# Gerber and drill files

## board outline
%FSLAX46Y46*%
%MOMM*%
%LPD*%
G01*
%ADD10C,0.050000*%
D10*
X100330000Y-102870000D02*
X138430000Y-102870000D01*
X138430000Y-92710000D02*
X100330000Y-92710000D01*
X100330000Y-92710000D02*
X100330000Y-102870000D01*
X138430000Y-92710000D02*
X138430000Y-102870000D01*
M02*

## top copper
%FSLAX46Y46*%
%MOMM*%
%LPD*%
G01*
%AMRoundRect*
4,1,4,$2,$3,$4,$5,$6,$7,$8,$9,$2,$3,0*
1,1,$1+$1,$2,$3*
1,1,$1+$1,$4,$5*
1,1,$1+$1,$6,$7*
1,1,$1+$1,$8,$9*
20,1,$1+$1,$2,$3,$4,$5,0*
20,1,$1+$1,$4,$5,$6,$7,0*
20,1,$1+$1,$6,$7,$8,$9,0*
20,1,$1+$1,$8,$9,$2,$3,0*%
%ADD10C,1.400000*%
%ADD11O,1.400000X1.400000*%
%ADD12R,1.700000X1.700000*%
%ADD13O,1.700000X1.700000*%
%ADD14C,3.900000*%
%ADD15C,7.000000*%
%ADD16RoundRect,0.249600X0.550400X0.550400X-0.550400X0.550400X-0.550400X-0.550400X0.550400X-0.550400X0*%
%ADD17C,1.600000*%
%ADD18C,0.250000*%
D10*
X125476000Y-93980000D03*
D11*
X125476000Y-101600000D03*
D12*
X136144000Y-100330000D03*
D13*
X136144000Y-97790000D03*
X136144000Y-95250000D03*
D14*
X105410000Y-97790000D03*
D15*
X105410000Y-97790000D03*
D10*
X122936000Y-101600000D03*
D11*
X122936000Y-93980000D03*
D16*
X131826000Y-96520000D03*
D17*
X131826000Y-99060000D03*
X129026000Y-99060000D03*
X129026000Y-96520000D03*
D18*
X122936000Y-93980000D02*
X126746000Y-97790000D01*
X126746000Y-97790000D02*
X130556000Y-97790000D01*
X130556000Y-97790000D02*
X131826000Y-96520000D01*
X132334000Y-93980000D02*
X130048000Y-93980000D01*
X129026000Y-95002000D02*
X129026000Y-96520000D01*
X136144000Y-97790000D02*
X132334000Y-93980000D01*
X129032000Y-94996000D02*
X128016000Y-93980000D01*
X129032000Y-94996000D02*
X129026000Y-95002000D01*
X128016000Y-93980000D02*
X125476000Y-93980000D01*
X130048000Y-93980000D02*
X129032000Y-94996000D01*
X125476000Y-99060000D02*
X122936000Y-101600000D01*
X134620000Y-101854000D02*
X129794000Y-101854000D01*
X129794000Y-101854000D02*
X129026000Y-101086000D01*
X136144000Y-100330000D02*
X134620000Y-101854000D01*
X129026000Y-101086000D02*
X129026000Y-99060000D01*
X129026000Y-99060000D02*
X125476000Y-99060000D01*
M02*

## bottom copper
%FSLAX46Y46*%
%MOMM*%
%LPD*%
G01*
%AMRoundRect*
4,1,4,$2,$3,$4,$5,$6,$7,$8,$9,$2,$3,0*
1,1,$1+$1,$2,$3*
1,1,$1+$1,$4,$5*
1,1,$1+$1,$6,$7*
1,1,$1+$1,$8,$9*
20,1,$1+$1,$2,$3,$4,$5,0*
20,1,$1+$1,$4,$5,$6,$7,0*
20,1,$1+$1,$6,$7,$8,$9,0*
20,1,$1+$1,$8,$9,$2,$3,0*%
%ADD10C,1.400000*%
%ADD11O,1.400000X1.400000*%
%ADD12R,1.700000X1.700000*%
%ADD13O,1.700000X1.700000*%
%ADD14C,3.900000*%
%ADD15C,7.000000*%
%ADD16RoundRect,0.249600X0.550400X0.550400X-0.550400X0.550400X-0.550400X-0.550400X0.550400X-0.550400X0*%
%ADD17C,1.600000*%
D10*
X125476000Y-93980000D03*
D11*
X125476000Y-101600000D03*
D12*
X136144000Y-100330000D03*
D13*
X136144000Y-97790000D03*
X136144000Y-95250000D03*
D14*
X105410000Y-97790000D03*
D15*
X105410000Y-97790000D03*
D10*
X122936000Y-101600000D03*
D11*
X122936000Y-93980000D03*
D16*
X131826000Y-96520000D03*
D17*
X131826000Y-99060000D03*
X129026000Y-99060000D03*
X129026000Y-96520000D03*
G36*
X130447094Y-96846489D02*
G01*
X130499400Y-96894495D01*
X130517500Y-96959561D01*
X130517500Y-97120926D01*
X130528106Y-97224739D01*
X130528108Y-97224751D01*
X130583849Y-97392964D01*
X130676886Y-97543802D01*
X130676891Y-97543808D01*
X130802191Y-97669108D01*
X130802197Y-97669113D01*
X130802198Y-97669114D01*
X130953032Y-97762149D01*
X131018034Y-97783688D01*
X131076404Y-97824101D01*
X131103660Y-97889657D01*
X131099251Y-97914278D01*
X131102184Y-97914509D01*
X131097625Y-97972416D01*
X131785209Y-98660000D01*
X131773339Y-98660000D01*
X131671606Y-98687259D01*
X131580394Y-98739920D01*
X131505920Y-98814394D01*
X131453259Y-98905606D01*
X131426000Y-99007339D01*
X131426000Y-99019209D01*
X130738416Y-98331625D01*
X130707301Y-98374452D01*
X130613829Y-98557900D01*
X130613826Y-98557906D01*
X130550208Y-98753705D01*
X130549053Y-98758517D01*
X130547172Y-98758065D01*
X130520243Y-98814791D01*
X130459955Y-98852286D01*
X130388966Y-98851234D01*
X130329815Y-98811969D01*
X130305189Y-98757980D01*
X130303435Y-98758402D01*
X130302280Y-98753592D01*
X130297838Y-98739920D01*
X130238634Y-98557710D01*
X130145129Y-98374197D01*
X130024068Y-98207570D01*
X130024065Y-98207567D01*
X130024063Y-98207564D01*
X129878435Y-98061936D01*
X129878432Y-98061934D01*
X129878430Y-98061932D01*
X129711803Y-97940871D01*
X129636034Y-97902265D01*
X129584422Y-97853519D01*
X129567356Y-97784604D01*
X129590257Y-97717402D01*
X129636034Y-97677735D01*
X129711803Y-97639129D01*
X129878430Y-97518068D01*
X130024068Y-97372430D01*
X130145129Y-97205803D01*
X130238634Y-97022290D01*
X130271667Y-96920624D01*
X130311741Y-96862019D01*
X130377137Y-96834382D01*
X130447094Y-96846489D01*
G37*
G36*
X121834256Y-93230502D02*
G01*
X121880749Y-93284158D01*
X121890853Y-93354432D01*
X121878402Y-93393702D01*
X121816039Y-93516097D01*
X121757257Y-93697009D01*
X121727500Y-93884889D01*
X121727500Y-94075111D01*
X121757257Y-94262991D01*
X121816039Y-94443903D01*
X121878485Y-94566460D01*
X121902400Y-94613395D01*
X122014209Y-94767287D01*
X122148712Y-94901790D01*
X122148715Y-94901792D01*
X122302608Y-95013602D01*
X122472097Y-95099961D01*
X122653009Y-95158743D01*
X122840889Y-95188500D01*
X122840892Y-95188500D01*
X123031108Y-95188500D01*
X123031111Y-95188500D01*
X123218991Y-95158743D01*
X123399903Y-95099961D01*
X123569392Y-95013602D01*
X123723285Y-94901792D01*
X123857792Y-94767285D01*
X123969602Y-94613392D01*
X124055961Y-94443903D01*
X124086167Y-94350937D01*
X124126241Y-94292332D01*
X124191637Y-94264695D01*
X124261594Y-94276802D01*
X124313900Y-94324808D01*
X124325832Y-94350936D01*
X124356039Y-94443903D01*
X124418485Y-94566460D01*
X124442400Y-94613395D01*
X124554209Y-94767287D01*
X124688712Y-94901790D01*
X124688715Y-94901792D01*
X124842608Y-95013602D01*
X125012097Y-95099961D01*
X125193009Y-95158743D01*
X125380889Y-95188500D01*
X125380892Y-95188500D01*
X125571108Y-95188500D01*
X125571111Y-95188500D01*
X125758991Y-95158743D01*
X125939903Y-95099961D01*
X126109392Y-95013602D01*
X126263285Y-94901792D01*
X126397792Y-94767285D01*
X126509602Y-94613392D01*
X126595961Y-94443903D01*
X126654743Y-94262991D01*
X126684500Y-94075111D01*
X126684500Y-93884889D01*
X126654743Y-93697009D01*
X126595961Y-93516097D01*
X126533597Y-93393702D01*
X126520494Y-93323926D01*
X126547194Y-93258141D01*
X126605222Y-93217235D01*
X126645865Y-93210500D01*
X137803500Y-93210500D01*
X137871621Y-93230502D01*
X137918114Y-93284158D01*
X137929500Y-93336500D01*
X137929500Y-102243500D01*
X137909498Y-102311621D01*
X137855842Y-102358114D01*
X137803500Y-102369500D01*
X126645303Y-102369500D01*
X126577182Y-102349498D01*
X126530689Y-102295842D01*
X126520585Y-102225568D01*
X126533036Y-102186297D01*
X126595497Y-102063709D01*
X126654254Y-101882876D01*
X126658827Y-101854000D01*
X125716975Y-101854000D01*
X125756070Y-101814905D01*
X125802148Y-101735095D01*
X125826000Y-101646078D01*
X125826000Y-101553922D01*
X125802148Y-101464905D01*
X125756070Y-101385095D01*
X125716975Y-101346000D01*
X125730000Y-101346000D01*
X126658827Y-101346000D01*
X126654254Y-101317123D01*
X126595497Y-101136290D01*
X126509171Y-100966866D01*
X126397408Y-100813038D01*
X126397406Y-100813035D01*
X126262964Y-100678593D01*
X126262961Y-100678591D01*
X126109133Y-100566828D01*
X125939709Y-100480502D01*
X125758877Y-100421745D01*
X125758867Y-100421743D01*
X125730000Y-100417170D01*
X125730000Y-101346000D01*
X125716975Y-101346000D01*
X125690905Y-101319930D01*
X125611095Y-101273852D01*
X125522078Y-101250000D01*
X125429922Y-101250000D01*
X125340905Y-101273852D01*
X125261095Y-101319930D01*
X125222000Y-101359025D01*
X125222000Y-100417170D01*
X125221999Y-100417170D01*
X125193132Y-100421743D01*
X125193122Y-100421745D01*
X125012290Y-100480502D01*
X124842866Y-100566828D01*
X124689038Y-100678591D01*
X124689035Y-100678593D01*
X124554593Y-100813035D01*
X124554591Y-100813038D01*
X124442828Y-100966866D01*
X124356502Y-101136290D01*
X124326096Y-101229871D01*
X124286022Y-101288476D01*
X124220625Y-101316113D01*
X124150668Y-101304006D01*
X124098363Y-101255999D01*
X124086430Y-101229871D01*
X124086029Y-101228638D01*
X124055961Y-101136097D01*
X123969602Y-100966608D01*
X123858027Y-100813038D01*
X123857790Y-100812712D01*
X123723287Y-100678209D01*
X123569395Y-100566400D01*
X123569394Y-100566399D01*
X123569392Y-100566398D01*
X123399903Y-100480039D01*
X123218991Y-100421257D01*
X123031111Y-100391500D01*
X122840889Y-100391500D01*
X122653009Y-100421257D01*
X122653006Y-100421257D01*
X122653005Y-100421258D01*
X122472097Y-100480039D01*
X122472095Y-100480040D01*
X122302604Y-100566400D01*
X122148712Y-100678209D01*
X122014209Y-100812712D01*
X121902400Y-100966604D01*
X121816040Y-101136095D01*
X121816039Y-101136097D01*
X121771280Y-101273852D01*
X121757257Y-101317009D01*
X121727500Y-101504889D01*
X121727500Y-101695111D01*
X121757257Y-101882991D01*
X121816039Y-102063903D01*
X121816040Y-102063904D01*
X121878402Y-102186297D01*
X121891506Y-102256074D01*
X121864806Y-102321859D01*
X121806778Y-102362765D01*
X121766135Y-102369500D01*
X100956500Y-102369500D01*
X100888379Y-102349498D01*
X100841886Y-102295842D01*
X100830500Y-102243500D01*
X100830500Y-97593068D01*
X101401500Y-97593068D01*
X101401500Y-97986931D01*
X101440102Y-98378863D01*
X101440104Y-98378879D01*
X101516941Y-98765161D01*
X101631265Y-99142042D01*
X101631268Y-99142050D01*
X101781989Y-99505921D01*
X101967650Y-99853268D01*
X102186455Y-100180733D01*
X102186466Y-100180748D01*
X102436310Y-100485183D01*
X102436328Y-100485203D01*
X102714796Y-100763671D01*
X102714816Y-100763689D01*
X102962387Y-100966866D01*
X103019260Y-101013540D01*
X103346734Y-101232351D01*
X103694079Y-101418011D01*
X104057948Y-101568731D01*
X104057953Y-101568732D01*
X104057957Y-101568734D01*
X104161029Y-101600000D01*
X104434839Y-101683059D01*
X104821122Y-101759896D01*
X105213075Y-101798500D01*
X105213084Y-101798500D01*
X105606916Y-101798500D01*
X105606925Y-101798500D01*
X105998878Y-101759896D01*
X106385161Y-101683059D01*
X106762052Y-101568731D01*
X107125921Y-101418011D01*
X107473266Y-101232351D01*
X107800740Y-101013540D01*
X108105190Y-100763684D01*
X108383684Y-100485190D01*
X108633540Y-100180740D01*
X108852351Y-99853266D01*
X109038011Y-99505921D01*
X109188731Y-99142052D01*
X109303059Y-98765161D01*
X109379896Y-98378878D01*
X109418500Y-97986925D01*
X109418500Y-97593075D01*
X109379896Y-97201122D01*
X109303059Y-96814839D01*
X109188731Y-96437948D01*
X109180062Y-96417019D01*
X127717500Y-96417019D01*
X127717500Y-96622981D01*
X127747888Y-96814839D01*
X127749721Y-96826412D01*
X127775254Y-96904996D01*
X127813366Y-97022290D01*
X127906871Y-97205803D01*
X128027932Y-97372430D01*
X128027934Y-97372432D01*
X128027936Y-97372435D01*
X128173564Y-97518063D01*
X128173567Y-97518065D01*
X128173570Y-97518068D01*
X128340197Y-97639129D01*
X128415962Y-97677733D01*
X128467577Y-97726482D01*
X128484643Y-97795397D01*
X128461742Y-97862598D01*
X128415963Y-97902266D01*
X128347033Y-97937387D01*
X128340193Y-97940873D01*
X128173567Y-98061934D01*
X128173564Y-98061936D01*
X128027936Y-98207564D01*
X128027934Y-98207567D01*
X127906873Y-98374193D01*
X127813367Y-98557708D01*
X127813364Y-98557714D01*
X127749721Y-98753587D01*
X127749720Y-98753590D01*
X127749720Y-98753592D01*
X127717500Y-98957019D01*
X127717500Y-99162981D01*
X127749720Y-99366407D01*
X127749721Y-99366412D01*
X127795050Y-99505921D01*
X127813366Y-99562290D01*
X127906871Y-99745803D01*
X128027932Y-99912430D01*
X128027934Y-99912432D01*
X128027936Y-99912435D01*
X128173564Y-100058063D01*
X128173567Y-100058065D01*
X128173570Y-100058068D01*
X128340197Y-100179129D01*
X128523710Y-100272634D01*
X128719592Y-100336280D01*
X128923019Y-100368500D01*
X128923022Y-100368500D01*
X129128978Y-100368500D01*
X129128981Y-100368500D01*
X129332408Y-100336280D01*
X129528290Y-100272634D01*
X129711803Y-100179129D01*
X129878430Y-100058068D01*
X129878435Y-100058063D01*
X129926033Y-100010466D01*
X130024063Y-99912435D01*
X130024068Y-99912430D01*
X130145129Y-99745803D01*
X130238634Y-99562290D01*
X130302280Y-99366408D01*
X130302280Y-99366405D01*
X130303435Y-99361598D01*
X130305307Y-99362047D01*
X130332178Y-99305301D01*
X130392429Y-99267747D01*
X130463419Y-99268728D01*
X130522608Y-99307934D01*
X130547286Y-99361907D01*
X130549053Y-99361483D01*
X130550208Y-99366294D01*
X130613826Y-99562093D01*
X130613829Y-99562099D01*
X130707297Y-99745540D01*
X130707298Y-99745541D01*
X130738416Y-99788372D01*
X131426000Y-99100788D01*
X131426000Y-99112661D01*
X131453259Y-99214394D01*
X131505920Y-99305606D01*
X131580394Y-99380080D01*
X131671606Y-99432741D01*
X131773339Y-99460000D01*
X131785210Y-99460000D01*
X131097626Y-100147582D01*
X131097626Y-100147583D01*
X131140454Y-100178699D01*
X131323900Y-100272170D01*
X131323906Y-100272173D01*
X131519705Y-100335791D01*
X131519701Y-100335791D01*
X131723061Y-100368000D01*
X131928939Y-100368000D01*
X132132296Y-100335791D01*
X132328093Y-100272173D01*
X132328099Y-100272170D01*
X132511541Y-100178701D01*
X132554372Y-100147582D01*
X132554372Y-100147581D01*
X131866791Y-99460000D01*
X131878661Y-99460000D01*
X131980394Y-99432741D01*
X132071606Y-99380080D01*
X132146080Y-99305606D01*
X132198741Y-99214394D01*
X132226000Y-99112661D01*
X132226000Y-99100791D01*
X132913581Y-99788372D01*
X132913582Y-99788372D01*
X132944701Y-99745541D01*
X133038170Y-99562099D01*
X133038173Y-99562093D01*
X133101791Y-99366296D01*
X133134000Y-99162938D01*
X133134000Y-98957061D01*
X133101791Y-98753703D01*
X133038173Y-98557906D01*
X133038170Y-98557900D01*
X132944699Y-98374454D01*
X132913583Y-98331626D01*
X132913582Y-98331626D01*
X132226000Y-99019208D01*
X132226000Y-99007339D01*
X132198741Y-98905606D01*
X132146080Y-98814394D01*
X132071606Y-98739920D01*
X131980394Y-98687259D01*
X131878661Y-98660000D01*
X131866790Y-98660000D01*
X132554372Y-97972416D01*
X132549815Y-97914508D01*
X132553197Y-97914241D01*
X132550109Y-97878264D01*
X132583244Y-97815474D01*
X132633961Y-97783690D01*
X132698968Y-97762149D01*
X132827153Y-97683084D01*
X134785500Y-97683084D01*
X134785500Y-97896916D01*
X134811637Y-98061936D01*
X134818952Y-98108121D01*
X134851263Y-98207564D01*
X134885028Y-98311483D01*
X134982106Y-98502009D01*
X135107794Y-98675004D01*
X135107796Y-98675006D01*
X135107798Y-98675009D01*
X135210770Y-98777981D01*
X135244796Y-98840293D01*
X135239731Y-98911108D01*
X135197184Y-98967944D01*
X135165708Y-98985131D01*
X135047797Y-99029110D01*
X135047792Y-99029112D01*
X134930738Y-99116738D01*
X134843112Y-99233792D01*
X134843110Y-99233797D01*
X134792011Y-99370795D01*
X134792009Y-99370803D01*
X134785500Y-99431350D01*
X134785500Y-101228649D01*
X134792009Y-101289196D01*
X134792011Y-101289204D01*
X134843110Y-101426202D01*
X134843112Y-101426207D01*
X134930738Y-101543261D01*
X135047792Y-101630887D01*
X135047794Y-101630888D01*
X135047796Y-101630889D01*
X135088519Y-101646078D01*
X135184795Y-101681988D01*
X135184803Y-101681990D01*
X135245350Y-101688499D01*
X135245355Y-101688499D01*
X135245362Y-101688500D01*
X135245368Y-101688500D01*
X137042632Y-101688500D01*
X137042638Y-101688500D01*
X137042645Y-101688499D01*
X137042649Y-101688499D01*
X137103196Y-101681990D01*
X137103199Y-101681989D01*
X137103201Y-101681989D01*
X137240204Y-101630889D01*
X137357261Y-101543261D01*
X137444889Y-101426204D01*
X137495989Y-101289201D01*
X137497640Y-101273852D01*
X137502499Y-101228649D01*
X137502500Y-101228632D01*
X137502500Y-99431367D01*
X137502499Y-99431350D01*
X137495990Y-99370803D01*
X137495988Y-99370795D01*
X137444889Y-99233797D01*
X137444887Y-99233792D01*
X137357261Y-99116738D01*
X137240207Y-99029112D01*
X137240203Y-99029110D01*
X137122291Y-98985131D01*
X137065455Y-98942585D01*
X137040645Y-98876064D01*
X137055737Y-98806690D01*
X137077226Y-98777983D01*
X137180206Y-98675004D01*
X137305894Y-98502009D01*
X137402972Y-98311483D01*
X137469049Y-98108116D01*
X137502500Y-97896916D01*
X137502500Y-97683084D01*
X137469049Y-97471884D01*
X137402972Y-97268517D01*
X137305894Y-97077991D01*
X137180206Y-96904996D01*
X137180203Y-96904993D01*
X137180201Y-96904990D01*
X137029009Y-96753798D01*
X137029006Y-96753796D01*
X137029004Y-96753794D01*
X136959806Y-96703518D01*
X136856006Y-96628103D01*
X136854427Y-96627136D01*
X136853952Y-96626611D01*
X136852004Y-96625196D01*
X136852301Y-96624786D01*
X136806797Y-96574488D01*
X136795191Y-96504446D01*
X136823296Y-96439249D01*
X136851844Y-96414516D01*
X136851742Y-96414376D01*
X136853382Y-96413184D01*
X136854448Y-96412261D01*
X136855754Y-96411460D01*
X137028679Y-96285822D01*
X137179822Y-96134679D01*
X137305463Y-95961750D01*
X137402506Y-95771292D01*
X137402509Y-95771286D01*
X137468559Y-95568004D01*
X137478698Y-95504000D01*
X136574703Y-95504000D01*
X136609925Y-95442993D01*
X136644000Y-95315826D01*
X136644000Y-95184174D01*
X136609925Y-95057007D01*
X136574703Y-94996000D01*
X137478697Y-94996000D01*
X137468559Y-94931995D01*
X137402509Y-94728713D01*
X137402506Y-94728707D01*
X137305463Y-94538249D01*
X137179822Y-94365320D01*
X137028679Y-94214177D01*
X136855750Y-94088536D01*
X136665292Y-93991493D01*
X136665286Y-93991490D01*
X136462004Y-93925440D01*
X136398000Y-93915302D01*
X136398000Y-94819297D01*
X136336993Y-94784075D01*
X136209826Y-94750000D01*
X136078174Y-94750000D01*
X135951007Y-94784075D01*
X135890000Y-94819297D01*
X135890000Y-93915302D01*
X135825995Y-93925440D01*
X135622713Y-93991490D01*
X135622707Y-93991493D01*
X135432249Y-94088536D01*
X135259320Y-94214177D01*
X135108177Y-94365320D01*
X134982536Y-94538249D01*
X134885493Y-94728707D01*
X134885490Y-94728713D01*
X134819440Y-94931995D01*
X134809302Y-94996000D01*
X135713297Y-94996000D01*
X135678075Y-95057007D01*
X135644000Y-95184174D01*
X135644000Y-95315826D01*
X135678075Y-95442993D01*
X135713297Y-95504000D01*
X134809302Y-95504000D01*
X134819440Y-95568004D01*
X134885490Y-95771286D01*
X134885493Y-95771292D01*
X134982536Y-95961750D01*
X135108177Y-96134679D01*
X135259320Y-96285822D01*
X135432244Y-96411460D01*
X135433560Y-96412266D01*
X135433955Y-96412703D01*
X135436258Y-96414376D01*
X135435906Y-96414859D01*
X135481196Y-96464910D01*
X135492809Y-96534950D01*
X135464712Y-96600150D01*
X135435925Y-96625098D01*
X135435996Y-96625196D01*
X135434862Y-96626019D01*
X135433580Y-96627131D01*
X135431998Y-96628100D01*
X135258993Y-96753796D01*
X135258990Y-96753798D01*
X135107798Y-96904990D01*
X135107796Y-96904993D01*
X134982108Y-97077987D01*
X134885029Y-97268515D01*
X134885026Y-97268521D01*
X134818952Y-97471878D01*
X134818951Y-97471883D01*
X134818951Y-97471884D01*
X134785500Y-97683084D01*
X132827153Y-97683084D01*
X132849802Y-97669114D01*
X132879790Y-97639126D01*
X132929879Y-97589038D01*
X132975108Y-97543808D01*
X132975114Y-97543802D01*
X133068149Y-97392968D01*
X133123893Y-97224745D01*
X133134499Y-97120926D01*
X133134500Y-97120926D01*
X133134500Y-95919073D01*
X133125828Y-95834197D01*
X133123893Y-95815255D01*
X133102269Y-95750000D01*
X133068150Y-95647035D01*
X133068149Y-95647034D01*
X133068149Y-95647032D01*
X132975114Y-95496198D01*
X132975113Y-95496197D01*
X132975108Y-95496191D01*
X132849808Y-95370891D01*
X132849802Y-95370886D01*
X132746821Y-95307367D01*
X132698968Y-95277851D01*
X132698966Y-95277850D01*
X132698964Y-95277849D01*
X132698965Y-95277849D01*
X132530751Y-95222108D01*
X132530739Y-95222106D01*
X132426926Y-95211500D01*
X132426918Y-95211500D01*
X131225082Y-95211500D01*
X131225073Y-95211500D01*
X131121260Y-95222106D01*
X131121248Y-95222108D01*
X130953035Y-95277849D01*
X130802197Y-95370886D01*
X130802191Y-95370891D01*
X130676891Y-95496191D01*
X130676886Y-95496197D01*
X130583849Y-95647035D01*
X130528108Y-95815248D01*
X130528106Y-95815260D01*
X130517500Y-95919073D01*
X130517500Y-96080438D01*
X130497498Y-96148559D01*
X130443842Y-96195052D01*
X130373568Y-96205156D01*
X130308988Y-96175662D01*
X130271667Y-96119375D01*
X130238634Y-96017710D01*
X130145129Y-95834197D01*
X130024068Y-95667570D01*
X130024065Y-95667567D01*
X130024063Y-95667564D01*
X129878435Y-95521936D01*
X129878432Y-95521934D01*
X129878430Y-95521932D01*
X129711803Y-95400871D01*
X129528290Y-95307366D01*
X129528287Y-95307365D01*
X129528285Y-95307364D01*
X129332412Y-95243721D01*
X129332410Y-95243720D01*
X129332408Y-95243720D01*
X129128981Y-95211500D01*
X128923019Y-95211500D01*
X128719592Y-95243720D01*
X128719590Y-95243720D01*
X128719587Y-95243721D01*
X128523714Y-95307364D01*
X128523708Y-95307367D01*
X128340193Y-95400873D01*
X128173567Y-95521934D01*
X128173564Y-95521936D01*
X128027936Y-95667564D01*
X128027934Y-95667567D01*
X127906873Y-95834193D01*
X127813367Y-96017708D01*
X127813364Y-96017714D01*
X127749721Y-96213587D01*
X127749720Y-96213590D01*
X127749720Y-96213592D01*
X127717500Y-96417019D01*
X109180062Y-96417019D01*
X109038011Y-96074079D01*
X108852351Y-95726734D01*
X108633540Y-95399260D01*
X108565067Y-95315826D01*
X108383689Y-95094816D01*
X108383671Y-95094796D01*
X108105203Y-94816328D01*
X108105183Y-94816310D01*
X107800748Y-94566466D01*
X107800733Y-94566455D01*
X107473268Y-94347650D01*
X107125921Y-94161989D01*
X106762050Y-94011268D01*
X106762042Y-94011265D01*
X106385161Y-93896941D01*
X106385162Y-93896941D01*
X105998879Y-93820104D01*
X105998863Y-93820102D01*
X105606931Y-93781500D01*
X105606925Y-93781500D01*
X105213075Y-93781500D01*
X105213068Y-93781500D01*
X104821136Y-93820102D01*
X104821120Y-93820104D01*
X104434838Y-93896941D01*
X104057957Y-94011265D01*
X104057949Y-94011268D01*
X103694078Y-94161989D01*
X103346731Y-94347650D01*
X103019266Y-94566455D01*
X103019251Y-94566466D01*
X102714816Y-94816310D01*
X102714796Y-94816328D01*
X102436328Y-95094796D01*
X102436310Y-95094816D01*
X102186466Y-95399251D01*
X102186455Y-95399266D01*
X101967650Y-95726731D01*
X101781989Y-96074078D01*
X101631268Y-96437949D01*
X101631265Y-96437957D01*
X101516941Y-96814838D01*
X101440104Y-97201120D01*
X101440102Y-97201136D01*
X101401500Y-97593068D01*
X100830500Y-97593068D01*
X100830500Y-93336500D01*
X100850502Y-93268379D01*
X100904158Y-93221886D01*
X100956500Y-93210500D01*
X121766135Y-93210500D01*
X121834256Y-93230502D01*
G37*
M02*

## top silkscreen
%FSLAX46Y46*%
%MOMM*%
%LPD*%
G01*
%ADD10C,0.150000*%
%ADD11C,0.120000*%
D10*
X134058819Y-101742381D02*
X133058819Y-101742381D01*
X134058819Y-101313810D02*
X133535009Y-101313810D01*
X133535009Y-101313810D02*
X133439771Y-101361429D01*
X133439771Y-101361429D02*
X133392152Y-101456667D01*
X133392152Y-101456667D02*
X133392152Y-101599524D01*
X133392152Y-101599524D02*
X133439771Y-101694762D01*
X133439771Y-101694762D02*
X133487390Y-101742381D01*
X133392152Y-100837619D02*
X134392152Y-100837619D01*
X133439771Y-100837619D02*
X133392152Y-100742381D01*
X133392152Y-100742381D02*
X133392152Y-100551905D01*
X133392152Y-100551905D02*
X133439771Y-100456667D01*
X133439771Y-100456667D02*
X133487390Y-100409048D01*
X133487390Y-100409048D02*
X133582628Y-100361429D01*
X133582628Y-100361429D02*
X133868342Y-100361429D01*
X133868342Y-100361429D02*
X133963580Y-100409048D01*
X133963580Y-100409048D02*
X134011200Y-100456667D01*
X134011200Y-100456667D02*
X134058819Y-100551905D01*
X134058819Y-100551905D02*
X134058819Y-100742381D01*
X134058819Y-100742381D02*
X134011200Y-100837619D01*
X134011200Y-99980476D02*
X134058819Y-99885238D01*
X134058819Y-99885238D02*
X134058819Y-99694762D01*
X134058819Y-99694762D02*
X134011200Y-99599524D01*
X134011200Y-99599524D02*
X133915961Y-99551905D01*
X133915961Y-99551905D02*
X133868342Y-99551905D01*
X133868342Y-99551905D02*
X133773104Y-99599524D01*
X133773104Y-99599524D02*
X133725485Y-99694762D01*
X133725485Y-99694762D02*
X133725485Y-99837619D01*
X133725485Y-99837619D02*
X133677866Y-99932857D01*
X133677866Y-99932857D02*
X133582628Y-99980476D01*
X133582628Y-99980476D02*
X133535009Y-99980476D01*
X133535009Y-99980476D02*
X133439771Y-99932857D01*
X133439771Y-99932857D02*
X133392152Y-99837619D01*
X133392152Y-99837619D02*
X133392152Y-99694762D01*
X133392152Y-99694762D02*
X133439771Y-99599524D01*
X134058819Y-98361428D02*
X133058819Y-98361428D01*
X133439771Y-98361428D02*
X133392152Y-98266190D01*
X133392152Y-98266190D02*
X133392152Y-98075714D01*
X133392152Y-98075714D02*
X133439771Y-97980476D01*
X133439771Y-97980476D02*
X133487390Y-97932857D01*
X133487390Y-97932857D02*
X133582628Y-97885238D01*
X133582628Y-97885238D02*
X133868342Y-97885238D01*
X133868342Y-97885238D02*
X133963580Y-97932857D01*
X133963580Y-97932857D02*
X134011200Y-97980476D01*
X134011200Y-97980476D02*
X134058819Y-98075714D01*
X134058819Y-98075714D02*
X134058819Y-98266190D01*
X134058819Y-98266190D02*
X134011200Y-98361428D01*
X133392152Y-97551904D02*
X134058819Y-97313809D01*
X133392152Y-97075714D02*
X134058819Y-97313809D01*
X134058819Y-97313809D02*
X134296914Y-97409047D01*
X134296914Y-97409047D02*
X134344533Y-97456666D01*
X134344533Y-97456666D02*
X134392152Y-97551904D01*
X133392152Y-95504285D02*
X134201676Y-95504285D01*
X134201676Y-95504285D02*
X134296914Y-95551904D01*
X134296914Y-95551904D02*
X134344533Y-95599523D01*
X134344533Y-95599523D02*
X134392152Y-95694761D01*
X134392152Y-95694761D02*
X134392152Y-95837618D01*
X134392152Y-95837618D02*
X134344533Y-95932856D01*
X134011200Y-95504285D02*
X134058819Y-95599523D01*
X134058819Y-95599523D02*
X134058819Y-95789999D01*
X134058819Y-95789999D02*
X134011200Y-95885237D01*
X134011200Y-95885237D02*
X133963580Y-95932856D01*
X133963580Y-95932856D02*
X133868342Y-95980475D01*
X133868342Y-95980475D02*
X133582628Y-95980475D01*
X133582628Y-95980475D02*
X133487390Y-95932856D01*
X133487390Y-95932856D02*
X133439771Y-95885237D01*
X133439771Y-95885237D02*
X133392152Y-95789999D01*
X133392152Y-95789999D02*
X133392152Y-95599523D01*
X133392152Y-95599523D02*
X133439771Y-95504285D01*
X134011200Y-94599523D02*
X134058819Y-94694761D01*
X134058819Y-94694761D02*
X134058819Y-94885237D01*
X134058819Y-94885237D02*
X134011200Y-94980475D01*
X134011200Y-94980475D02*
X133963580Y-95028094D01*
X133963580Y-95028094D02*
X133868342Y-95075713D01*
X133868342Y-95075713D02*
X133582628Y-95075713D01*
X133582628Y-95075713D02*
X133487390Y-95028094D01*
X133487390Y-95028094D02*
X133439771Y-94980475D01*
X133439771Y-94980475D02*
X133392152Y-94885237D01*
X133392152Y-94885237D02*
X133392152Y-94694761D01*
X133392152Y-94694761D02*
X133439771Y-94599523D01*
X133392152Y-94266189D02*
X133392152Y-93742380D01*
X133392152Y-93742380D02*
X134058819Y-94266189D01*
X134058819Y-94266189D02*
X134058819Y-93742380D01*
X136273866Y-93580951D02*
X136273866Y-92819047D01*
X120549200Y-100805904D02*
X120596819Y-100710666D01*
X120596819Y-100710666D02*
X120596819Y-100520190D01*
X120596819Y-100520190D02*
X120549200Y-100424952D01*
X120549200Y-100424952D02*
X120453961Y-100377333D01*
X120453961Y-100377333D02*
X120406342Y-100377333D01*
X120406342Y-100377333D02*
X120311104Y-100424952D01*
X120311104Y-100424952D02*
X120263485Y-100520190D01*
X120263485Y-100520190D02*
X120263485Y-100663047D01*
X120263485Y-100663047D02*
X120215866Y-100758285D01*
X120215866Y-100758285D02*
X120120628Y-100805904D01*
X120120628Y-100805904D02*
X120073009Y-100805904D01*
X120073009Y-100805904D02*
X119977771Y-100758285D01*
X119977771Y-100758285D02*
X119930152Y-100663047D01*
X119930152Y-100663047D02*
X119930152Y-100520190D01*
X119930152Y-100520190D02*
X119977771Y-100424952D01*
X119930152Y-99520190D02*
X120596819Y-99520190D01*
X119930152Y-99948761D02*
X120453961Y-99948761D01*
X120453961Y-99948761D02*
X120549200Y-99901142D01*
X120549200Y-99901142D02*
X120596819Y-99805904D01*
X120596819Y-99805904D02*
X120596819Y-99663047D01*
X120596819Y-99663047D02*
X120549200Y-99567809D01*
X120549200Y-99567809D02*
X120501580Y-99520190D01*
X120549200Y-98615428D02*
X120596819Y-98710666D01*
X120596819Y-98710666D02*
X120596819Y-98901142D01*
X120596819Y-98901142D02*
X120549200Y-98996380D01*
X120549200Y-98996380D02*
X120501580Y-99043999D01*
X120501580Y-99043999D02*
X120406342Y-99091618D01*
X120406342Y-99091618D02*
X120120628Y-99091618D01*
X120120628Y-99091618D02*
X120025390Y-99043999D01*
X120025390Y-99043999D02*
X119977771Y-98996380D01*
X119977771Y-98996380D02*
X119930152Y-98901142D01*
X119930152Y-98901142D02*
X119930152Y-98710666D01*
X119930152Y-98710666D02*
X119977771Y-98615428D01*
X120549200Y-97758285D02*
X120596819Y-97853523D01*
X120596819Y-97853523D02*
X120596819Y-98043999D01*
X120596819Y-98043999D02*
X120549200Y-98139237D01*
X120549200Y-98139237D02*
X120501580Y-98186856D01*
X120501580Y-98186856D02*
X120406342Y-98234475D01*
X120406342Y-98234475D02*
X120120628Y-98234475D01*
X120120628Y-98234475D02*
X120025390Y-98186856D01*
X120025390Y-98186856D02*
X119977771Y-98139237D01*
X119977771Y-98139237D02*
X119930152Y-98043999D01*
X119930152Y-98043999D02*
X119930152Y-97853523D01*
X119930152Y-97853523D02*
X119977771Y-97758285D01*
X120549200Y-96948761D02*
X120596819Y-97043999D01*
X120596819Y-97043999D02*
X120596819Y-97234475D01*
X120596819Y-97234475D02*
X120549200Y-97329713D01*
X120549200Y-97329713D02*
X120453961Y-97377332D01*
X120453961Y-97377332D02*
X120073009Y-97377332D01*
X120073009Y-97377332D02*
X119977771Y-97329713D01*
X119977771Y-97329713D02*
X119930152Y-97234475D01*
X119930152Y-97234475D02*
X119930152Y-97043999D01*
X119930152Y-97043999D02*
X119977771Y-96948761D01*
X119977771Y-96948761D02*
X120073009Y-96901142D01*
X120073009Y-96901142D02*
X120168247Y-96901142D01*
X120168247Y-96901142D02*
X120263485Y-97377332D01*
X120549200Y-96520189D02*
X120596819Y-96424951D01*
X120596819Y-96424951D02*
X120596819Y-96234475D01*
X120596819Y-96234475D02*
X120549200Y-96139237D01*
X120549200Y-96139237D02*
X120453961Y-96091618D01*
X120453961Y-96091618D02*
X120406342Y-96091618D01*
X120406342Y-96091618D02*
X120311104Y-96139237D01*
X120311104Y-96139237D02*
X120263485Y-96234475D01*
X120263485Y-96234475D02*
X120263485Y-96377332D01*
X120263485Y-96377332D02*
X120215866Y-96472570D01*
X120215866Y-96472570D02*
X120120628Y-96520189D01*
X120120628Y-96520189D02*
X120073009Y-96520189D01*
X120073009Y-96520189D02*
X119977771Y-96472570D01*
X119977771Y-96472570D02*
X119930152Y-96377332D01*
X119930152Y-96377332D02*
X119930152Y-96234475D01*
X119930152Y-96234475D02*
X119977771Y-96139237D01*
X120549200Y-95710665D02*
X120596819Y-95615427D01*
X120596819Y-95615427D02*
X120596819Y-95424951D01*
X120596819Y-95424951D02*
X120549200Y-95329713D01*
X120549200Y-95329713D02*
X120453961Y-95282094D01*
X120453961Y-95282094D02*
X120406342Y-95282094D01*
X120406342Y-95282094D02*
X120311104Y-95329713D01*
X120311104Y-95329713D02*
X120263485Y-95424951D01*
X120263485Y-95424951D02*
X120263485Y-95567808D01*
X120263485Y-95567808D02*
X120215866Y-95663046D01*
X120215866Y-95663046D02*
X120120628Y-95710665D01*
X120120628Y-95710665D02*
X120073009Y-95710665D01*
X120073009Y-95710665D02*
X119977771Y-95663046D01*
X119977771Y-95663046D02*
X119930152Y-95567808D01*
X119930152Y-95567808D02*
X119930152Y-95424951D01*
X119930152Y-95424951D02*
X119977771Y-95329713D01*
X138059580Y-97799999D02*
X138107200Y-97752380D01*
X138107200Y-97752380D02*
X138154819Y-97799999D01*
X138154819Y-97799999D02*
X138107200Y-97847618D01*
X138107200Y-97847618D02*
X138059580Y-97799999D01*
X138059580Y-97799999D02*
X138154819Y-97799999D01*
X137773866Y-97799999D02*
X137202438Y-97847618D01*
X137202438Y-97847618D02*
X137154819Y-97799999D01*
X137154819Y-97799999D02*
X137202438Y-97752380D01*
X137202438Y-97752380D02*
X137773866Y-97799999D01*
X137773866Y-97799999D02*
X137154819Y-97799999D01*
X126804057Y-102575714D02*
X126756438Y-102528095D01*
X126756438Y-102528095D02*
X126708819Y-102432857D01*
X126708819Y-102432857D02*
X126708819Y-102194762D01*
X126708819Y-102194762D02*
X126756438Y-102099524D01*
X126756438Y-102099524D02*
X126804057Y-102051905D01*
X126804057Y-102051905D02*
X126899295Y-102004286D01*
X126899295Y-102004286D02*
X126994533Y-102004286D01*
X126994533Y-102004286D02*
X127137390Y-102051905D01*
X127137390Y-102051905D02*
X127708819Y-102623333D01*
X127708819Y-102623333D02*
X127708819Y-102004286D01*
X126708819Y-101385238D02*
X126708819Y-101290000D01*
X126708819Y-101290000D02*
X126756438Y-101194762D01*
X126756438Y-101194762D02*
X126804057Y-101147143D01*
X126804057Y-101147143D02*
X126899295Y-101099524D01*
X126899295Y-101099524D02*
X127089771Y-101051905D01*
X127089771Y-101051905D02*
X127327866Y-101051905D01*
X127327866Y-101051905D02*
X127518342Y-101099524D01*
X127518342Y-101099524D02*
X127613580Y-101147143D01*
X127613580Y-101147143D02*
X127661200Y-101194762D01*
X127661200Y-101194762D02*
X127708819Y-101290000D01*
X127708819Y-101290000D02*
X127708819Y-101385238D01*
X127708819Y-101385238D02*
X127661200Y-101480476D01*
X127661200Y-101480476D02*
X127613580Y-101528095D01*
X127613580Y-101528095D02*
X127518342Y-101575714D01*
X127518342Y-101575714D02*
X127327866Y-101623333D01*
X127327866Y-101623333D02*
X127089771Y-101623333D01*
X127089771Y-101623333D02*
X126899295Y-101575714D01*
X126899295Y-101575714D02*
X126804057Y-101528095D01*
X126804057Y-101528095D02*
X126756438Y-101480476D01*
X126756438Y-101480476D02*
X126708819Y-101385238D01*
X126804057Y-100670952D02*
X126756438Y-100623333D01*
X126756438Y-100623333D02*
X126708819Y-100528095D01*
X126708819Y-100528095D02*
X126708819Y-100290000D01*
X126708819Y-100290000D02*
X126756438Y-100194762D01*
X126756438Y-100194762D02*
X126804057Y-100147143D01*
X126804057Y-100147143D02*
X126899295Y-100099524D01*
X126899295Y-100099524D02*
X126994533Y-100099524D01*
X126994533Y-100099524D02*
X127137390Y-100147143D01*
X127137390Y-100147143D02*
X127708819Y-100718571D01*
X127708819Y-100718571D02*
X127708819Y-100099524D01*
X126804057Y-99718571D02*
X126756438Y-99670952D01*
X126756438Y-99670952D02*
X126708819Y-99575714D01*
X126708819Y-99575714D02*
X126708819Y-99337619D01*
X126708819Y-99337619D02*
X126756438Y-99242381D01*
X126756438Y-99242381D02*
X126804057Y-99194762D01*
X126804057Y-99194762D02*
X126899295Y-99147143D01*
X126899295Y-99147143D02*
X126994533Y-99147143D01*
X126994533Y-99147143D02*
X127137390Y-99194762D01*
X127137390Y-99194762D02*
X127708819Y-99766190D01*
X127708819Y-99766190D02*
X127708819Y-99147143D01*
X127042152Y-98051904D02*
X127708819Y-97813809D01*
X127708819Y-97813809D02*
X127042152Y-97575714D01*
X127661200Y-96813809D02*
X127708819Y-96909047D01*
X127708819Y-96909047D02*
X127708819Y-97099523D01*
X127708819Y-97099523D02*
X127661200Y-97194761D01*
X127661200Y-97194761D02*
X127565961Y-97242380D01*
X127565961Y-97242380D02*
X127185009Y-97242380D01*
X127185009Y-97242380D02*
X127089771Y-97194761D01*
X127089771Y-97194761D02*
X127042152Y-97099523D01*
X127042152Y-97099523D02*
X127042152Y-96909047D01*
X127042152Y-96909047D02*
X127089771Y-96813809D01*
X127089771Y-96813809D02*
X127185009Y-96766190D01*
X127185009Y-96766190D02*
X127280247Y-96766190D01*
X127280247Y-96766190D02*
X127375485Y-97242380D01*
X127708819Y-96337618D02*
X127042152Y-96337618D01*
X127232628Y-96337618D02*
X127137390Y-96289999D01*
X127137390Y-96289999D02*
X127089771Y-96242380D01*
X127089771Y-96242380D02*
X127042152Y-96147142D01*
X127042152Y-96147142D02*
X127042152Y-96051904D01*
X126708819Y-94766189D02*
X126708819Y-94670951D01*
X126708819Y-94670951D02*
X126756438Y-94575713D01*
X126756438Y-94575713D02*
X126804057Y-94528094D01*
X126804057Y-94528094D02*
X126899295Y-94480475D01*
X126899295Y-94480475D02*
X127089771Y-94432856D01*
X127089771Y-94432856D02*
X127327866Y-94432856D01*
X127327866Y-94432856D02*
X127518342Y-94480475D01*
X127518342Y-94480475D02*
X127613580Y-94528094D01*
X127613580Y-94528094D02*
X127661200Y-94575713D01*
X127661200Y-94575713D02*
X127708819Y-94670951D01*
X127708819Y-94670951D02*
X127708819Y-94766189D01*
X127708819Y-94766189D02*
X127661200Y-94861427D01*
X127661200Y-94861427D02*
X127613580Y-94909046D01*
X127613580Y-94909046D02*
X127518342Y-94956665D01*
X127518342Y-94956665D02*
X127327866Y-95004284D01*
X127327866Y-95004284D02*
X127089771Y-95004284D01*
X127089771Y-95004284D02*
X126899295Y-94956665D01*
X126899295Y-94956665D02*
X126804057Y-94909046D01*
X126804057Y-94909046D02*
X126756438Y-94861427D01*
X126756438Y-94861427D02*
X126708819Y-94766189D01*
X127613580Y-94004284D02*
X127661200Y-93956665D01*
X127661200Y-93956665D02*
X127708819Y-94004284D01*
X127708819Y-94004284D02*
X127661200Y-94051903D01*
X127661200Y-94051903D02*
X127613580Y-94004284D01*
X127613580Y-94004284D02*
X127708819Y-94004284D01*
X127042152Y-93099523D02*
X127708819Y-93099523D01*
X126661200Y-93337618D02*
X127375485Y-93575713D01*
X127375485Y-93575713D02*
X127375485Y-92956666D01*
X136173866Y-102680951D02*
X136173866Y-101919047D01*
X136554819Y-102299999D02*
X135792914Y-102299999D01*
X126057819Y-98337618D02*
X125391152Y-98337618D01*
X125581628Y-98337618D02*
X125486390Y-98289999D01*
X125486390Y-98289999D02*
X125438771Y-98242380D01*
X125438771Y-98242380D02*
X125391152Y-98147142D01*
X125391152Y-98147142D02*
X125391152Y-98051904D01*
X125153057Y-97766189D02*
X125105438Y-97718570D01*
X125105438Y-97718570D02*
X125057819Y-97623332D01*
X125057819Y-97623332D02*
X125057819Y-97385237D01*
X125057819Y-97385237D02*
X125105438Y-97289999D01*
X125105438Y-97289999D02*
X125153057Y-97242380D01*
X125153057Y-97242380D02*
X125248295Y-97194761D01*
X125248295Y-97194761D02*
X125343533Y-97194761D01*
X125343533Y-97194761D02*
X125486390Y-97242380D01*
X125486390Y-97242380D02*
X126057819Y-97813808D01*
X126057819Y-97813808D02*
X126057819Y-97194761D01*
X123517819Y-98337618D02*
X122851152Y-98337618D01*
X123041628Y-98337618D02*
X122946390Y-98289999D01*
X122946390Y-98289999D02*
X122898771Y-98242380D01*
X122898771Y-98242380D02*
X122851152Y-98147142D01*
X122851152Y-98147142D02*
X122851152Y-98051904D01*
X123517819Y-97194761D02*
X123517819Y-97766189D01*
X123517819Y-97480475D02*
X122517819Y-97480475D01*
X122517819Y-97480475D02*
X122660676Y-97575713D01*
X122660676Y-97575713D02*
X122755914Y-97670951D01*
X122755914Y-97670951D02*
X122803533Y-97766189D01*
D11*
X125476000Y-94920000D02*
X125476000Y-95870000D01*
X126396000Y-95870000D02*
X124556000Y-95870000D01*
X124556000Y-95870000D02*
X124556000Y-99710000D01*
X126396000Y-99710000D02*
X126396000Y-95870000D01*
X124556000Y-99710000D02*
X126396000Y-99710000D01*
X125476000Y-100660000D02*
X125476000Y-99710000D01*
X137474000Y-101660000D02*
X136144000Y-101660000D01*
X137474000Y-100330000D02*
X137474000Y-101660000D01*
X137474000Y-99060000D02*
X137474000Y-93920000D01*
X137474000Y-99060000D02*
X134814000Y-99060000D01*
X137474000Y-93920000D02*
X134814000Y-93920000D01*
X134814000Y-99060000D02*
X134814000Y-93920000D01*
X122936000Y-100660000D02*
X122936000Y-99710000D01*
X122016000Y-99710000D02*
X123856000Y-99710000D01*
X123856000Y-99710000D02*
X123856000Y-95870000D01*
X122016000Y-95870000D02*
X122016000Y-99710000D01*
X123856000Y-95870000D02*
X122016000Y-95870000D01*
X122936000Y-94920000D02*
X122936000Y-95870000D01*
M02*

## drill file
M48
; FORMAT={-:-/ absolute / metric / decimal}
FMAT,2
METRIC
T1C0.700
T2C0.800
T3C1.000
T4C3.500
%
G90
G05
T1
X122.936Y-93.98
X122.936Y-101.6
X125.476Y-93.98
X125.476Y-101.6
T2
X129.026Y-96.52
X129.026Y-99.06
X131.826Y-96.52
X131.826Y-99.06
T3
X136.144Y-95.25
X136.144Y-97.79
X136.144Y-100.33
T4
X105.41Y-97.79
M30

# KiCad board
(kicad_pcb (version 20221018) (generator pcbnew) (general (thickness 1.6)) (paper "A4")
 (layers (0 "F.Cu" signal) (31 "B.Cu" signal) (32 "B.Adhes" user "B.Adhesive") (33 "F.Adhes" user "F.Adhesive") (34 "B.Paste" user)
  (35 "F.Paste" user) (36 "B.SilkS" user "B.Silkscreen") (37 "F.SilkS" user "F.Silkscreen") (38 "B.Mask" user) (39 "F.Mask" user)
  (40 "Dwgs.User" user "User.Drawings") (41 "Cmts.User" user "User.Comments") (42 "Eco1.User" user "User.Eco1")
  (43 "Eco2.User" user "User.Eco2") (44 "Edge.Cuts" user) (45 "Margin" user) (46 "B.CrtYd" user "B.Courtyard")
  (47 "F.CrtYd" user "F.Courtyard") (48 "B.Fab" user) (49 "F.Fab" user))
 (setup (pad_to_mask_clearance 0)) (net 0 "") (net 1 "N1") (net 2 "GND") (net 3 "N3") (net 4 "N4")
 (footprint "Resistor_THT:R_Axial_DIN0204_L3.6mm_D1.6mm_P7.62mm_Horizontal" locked (layer "F.Cu") (at 125.476 93.98 -90)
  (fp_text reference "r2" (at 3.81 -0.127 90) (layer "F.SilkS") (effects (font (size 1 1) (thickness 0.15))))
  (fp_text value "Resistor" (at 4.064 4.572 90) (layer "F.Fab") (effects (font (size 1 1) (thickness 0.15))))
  (fp_line (start 0.94 0) (end 1.89 0) (stroke (width 0.12) (type solid)) (layer "F.SilkS"))
  (fp_line (start 1.89 -0.92) (end 1.89 0.92) (stroke (width 0.12) (type solid)) (layer "F.SilkS"))
  (fp_line (start 1.89 0.92) (end 5.73 0.92) (stroke (width 0.12) (type solid)) (layer "F.SilkS"))
  (fp_line (start 5.73 -0.92) (end 1.89 -0.92) (stroke (width 0.12) (type solid)) (layer "F.SilkS"))
  (fp_line (start 5.73 0.92) (end 5.73 -0.92) (stroke (width 0.12) (type solid)) (layer "F.SilkS"))
  (fp_line (start 6.68 0) (end 5.73 0) (stroke (width 0.12) (type solid)) (layer "F.SilkS"))
  (pad "1" thru_hole circle locked (at 0 0 270) (size 1.4 1.4) (drill 0.7) (layers "*.Cu" "*.Mask") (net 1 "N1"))
  (pad "2" thru_hole oval locked (at 7.62 0 270) (size 1.4 1.4) (drill 0.7) (layers "*.Cu" "*.Mask") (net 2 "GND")))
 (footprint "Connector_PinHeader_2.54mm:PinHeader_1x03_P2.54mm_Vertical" (layer "F.Cu") (at 136.144 100.33 180)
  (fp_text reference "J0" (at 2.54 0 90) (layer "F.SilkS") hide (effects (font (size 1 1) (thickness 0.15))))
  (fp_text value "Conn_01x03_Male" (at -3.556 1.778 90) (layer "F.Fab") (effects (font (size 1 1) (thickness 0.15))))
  (fp_line (start -1.33 -1.33) (end 0 -1.33) (stroke (width 0.12) (type solid)) (layer "F.SilkS"))
  (fp_line (start -1.33 0) (end -1.33 -1.33) (stroke (width 0.12) (type solid)) (layer "F.SilkS"))
  (fp_line (start -1.33 1.27) (end -1.33 6.41) (stroke (width 0.12) (type solid)) (layer "F.SilkS"))
  (fp_line (start -1.33 1.27) (end 1.33 1.27) (stroke (width 0.12) (type solid)) (layer "F.SilkS"))
  (fp_line (start -1.33 6.41) (end 1.33 6.41) (stroke (width 0.12) (type solid)) (layer "F.SilkS"))
  (fp_line (start 1.33 1.27) (end 1.33 6.41) (stroke (width 0.12) (type solid)) (layer "F.SilkS"))
  (pad "1" thru_hole rect (at 0 0 180) (size 1.7 1.7) (drill 1) (layers "*.Cu" "*.Mask") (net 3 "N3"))
  (pad "2" thru_hole oval (at 0 2.54 180) (size 1.7 1.7) (drill 1) (layers "*.Cu" "*.Mask") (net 1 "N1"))
  (pad "3" thru_hole oval (at 0 5.08 180) (size 1.7 1.7) (drill 1) (layers "*.Cu" "*.Mask") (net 2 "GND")))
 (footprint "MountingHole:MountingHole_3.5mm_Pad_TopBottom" (layer "F.Cu") (at 105.41 97.79)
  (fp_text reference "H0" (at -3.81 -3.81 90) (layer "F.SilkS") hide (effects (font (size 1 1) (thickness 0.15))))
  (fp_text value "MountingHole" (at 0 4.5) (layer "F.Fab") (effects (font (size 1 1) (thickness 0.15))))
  (pad "1" thru_hole circle (at 0 0) (size 3.9 3.9) (drill 3.5) (layers "*.Cu" "*.Mask"))
  (pad "1" connect circle (at 0 0) (size 7 7) (layers "F.Cu" "F.Mask"))
  (pad "1" connect circle (at 0 0) (size 7 7) (layers "B.Cu" "B.Mask")))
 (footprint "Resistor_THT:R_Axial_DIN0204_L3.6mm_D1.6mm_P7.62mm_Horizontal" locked (layer "F.Cu") (at 122.936 101.6 90)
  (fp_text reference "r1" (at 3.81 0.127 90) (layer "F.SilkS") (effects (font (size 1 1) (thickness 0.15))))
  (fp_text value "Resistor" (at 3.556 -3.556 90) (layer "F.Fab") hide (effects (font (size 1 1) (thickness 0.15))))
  (fp_line (start 0.94 0) (end 1.89 0) (stroke (width 0.12) (type solid)) (layer "F.SilkS"))
  (fp_line (start 1.89 -0.92) (end 1.89 0.92) (stroke (width 0.12) (type solid)) (layer "F.SilkS"))
  (fp_line (start 1.89 0.92) (end 5.73 0.92) (stroke (width 0.12) (type solid)) (layer "F.SilkS"))
  (fp_line (start 5.73 -0.92) (end 1.89 -0.92) (stroke (width 0.12) (type solid)) (layer "F.SilkS"))
  (fp_line (start 5.73 0.92) (end 5.73 -0.92) (stroke (width 0.12) (type solid)) (layer "F.SilkS"))
  (fp_line (start 6.68 0) (end 5.73 0) (stroke (width 0.12) (type solid)) (layer "F.SilkS"))
  (pad "1" thru_hole circle locked (at 0 0 90) (size 1.4 1.4) (drill 0.7) (layers "*.Cu" "*.Mask") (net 3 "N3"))
  (pad "2" thru_hole oval locked (at 7.62 0 90) (size 1.4 1.4) (drill 0.7) (layers "*.Cu" "*.Mask") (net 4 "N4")))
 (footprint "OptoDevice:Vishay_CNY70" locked (layer "B.Cu") (at 131.826 96.52 180)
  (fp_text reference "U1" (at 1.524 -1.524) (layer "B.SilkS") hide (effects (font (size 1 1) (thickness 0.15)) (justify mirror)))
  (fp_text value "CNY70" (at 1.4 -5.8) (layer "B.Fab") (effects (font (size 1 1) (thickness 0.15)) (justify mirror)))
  (pad "1" thru_hole roundrect locked (at 0 0 180) (size 1.6 1.6) (drill 0.8) (layers "*.Cu" "*.Mask") (roundrect_rratio 0.156) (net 4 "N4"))
  (pad "2" thru_hole circle locked (at 0 -2.54 180) (size 1.6 1.6) (drill 0.8) (layers "*.Cu" "*.Mask") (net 2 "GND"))
  (pad "3" thru_hole circle locked (at 2.8 -2.54 180) (size 1.6 1.6) (drill 0.8) (layers "*.Cu" "*.Mask") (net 3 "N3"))
  (pad "4" thru_hole circle locked (at 2.8 0 180) (size 1.6 1.6) (drill 0.8) (layers "*.Cu" "*.Mask") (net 1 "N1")))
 (gr_line (start 100.33 102.87) (end 138.43 102.87) (stroke (width 0.05) (type solid)) (layer "Edge.Cuts"))
 (gr_line (start 138.43 92.71) (end 100.33 92.71) (stroke (width 0.05) (type solid)) (layer "Edge.Cuts"))
 (gr_line (start 100.33 92.71) (end 100.33 102.87) (stroke (width 0.05) (type solid)) (layer "Edge.Cuts"))
 (gr_line (start 138.43 92.71) (end 138.43 102.87) (stroke (width 0.05) (type solid)) (layer "Edge.Cuts"))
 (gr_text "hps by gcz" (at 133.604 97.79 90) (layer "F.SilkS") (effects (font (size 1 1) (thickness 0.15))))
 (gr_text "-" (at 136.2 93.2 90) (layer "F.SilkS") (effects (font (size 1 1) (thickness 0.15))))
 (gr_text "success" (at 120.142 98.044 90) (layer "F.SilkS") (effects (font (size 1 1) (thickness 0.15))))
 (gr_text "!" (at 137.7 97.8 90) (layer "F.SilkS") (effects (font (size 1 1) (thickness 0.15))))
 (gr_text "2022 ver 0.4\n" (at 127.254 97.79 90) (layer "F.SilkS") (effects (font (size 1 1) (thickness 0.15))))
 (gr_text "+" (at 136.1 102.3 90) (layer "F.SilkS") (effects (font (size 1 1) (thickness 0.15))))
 (segment (start 122.936 93.98) (end 126.746 97.79) (width 0.25) (layer "F.Cu") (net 4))
 (segment (start 126.746 97.79) (end 130.556 97.79) (width 0.25) (layer "F.Cu") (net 4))
 (segment (start 130.556 97.79) (end 131.826 96.52) (width 0.25) (layer "F.Cu") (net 4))
 (segment (start 132.334 93.98) (end 130.048 93.98) (width 0.25) (layer "F.Cu") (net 1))
 (segment (start 129.026 95.002) (end 129.026 96.52) (width 0.25) (layer "F.Cu") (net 1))
 (segment (start 136.144 97.79) (end 132.334 93.98) (width 0.25) (layer "F.Cu") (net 1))
 (segment (start 129.032 94.996) (end 128.016 93.98) (width 0.25) (layer "F.Cu") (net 1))
 (segment (start 129.032 94.996) (end 129.026 95.002) (width 0.25) (layer "F.Cu") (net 1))
 (segment (start 128.016 93.98) (end 125.476 93.98) (width 0.25) (layer "F.Cu") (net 1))
 (segment (start 130.048 93.98) (end 129.032 94.996) (width 0.25) (layer "F.Cu") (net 1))
 (segment (start 125.476 99.06) (end 122.936 101.6) (width 0.25) (layer "F.Cu") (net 3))
 (segment (start 134.62 101.854) (end 129.794 101.854) (width 0.25) (layer "F.Cu") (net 3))
 (segment (start 129.794 101.854) (end 129.026 101.086) (width 0.25) (layer "F.Cu") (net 3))
 (segment (start 136.144 100.33) (end 134.62 101.854) (width 0.25) (layer "F.Cu") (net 3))
 (segment (start 129.026 101.086) (end 129.026 99.06) (width 0.25) (layer "F.Cu") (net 3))
 (segment (start 129.026 99.06) (end 125.476 99.06) (width 0.25) (layer "F.Cu") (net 3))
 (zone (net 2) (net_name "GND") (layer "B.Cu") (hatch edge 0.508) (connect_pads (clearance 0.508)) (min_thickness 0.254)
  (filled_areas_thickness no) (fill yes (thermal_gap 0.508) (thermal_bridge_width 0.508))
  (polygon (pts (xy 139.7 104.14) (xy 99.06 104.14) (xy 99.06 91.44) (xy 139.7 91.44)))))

